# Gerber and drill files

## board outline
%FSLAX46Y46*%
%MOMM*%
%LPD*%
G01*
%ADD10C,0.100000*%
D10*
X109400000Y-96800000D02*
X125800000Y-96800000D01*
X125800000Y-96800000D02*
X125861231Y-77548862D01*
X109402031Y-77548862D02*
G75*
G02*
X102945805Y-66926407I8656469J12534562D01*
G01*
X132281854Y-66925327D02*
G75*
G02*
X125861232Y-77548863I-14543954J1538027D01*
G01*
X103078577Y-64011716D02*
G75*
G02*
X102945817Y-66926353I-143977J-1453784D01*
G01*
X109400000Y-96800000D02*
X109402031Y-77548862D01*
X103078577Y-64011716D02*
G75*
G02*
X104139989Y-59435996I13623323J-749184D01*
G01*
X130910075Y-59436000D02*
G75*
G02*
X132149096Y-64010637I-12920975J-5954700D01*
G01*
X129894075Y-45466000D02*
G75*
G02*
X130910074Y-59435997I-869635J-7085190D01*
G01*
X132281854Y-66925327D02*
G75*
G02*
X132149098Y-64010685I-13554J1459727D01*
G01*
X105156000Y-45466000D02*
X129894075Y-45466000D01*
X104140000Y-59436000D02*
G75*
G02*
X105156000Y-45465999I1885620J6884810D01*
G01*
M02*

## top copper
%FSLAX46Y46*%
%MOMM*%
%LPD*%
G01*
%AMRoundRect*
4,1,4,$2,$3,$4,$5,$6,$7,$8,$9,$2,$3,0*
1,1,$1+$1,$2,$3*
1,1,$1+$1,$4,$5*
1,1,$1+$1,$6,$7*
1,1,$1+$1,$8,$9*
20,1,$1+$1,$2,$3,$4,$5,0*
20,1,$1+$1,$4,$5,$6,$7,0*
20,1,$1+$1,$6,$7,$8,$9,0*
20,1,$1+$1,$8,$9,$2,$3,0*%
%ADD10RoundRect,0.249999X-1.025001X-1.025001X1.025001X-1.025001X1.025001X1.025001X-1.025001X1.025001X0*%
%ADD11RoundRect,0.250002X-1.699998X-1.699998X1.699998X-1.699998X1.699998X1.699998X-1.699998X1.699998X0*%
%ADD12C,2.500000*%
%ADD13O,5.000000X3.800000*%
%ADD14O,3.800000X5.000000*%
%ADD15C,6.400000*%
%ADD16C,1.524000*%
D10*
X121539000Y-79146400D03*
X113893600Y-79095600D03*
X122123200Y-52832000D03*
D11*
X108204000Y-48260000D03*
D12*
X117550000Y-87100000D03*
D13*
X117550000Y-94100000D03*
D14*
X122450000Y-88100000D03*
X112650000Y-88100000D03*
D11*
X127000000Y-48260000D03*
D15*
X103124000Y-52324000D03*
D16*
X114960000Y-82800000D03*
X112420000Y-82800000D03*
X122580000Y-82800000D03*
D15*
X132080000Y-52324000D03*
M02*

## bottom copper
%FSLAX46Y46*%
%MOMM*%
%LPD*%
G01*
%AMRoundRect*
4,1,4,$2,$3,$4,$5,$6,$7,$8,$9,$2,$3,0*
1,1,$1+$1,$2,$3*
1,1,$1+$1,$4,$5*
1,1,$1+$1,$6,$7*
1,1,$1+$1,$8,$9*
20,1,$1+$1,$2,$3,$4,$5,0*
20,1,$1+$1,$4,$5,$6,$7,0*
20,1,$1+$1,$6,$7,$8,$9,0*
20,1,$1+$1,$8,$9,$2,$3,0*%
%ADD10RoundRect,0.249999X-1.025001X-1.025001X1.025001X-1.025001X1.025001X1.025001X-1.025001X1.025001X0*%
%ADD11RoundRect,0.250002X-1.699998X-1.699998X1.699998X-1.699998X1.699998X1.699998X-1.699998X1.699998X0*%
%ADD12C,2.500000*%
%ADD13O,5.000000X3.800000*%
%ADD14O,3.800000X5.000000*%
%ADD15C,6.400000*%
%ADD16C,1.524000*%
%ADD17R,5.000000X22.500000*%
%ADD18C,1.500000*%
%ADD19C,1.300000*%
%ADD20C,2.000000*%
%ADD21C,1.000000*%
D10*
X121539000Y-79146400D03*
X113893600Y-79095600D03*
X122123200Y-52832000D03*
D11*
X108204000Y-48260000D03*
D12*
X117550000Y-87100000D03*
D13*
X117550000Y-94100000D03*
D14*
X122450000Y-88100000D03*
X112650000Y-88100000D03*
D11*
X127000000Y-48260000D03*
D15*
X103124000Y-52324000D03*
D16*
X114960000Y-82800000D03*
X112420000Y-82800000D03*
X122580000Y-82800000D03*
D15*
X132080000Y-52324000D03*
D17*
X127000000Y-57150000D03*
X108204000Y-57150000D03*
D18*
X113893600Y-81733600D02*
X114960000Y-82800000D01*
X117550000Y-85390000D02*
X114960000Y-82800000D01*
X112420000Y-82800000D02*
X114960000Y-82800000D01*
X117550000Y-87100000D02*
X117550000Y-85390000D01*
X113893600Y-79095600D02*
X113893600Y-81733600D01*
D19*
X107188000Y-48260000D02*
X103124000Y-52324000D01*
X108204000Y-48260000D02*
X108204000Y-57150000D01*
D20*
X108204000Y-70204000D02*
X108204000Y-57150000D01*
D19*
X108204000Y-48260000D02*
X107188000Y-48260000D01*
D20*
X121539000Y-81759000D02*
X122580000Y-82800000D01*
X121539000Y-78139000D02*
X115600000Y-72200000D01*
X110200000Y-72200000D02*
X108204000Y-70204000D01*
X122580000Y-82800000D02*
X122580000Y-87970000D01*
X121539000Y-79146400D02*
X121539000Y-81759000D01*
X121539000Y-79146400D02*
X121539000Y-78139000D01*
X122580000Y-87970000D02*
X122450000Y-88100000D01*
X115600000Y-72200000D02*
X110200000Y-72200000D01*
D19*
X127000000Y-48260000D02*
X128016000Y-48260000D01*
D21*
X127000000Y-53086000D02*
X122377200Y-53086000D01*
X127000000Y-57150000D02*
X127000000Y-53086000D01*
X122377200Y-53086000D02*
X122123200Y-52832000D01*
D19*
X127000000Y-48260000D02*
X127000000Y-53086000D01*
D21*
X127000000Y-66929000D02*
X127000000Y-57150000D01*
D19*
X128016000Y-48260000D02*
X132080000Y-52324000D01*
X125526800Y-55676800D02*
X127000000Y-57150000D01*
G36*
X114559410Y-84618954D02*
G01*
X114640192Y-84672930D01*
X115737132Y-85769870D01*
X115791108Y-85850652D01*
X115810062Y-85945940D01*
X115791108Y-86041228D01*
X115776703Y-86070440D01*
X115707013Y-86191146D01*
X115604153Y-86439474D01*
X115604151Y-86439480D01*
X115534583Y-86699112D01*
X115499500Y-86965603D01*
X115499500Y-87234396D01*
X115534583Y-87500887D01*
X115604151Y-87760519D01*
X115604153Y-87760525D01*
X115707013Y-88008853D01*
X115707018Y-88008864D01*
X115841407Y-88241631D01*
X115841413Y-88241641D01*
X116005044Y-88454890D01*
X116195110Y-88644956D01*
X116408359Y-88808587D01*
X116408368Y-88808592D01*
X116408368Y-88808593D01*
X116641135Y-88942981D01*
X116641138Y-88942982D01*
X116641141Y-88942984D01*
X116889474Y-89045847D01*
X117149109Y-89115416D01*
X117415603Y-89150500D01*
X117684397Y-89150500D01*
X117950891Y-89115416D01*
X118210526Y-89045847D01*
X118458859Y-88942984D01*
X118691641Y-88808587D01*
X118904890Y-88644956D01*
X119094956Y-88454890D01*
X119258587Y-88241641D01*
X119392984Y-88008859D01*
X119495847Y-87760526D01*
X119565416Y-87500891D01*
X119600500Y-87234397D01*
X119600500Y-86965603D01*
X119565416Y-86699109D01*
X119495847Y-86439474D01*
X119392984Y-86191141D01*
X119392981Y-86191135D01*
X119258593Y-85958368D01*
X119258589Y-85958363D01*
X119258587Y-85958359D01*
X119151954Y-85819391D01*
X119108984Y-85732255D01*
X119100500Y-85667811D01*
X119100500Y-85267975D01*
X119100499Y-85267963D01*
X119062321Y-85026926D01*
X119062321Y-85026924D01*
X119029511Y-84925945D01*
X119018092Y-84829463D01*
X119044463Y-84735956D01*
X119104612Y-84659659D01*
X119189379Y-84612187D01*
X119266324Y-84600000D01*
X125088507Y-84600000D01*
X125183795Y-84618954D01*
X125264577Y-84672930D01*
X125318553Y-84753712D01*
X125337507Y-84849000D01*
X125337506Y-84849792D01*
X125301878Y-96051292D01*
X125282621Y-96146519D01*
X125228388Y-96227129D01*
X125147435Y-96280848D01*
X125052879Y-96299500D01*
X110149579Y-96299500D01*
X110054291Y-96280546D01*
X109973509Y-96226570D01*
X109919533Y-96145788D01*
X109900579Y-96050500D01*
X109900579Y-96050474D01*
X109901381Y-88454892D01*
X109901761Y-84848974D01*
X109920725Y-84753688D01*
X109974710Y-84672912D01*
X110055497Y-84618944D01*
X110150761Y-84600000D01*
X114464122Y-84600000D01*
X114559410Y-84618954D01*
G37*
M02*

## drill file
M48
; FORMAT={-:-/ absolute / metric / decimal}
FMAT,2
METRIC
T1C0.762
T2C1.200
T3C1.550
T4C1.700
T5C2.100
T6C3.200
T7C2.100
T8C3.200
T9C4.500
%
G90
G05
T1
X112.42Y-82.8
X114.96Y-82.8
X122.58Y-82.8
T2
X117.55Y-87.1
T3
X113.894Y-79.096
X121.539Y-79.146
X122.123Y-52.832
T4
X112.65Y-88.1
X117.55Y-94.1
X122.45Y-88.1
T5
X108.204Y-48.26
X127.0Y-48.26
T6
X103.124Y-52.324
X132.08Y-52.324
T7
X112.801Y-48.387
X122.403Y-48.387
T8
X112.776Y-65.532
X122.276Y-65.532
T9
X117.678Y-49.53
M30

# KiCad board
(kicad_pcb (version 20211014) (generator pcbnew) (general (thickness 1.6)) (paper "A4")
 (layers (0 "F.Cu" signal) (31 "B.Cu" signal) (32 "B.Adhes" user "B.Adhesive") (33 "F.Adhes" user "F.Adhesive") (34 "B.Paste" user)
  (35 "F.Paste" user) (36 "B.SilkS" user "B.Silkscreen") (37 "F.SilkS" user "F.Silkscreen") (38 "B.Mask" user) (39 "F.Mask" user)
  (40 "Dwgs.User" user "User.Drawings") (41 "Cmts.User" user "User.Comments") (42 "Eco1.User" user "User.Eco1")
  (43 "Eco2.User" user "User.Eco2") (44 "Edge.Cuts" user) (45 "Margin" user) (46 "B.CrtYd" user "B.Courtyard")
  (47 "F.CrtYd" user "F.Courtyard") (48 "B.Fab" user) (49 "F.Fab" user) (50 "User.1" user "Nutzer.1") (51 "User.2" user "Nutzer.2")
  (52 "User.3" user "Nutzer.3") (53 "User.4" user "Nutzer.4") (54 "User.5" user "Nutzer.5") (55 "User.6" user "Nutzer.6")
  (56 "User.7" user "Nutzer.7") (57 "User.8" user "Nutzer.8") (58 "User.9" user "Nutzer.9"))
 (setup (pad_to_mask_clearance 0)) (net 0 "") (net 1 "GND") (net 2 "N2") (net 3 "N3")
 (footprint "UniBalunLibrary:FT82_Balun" (layer "F.Cu") (at 117.602 65.532)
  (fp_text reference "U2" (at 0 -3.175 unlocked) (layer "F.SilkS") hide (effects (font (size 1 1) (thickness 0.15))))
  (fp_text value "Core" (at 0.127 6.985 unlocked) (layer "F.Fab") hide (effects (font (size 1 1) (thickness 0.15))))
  (pad "" np_thru_hole circle (at -4.826 0) (size 3.2 3.2) (drill 3.2) (layers *.Cu *.Mask))
  (pad "" np_thru_hole circle (at 4.6736 0) (size 3.2 3.2) (drill 3.2) (layers *.Cu *.Mask))
  (pad "1" thru_hole roundrect (at 3.937 13.6144) (size 2.55 2.55) (drill 1.55) (layers *.Cu *.Mask) (roundrect_rratio 0.098039)
   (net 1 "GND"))
  (pad "2" thru_hole roundrect (at -3.7084 13.5636) (size 2.55 2.55) (drill 1.55) (layers *.Cu *.Mask) (roundrect_rratio 0.098039)
   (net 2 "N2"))
  (pad "3" thru_hole roundrect (at 4.5212 -12.7) (size 2.55 2.55) (drill 1.55) (layers *.Cu *.Mask) (roundrect_rratio 0.098039) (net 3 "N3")))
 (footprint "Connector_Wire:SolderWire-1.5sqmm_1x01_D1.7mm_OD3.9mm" (layer "F.Cu") (at 108.204 48.26)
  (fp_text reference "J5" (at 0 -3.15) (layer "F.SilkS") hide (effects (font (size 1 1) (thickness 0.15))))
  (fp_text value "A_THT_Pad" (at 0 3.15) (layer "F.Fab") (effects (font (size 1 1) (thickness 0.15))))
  (pad "1" thru_hole roundrect (at 0 0) (size 3.9 3.9) (drill 2.1) (layers *.Cu *.Mask) (roundrect_rratio 0.064103) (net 1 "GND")))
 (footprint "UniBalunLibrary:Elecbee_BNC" (layer "F.Cu") (at 112.65 88.1)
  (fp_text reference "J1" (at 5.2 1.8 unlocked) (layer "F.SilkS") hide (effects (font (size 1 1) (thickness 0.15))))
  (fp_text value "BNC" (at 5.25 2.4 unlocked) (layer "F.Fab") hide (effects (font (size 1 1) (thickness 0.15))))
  (pad "1" thru_hole circle (at 4.9 -1) (size 2.5 2.5) (drill 1.2) (layers *.Cu *.Mask) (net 2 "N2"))
  (pad "2" thru_hole oval (at 4.9 6 90) (size 3.8 5) (drill 1.7) (layers *.Cu *.Mask) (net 1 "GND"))
  (pad "2" thru_hole oval (at 9.8 0) (size 3.8 5) (drill 1.7) (layers *.Cu *.Mask) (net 1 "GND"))
  (pad "2" thru_hole oval (at 0 0) (size 3.8 5) (drill 1.7) (layers *.Cu *.Mask) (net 1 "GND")))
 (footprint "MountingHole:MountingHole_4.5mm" (layer "F.Cu") (at 117.6782 49.53)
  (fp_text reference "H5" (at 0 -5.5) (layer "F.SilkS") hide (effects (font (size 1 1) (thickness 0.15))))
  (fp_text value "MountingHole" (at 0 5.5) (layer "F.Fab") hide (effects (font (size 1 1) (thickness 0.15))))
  (pad "" np_thru_hole circle (at 0 0) (size 4.5 4.5) (drill 4.5) (layers *.Cu *.Mask)))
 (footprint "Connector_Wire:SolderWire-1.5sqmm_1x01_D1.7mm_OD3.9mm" (layer "F.Cu") (at 127 48.26)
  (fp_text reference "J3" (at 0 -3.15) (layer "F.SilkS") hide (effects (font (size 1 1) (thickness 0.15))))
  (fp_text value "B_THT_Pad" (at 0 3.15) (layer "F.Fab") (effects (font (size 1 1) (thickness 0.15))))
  (pad "1" thru_hole roundrect (at 0 0) (size 3.9 3.9) (drill 2.1) (layers *.Cu *.Mask) (roundrect_rratio 0.064103) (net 3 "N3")))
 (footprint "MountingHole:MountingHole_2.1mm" (layer "F.Cu") (at 112.8014 48.387)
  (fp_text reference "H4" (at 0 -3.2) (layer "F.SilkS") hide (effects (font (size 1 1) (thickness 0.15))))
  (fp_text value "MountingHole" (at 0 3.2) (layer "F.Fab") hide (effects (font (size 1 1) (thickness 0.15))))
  (pad "" np_thru_hole circle (at 0 0) (size 2.1 2.1) (drill 2.1) (layers *.Cu *.Mask)))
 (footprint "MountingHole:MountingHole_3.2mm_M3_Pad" (layer "F.Cu") (at 103.124 52.324)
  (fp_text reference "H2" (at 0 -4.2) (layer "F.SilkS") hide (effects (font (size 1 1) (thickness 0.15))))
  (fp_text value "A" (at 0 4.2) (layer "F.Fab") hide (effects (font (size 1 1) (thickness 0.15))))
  (pad "1" thru_hole circle (at 0 0) (size 6.4 6.4) (drill 3.2) (layers *.Cu *.Mask) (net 1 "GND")))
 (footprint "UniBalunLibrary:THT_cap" (layer "F.Cu") (at 117.5 82.8)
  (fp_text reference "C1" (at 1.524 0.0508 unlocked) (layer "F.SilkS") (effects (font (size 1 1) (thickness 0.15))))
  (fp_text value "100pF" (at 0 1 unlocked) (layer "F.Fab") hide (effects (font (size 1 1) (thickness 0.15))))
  (pad "1" thru_hole circle (at -2.54 0) (size 1.524 1.524) (drill 0.762) (layers *.Cu *.Mask) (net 2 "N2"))
  (pad "1" thru_hole circle (at -5.08 0) (size 1.524 1.524) (drill 0.762) (layers *.Cu *.Mask) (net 2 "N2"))
  (pad "2" thru_hole circle (at 5.08 0) (size 1.524 1.524) (drill 0.762) (layers *.Cu *.Mask) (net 1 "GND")))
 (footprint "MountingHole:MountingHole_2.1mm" (layer "F.Cu") (at 122.4026 48.387)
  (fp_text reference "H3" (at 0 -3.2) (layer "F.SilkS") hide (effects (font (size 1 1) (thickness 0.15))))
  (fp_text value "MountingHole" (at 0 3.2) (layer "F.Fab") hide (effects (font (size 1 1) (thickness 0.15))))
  (pad "" np_thru_hole circle (at 0 0) (size 2.1 2.1) (drill 2.1) (layers *.Cu *.Mask)))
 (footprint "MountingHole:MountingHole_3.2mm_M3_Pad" (layer "F.Cu") (at 132.08 52.324)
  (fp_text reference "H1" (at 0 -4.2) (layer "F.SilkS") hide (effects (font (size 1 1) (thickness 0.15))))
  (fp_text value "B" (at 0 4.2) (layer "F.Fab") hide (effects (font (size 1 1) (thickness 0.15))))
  (pad "1" thru_hole circle (at 0 0) (size 6.4 6.4) (drill 3.2) (layers *.Cu *.Mask) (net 3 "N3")))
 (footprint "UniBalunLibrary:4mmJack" (layer "B.Cu") (at 127.254 56.896 90)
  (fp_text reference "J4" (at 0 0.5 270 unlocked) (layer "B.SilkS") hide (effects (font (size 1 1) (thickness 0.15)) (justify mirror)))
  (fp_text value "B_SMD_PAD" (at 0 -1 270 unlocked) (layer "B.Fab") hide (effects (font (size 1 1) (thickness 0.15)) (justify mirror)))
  (pad "1" smd rect (at -0.254 -0.254 90) (size 22.5 5) (layers "B.Cu" "B.Mask") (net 3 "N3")))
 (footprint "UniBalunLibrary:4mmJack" (layer "B.Cu") (at 108.458 56.896 90)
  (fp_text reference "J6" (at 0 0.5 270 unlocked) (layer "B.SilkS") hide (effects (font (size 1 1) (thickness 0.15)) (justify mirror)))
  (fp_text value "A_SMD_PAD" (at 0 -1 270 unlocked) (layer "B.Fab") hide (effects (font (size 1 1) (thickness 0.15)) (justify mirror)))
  (pad "1" smd rect (at -0.254 -0.254 90) (size 22.5 5) (layers "B.Cu" "B.Mask") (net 1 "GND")))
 (gr_line (start 109.4 96.8) (end 125.8 96.8) (layer "Edge.Cuts") (width 0.1))
 (gr_line (start 125.8 96.8) (end 125.861231 77.548862) (layer "Edge.Cuts") (width 0.1))
 (gr_arc (start 109.402031 77.548862) (mid 105.04112 72.92614) (end 102.945817 66.926406) (layer "Edge.Cuts") (width 0.1))
 (gr_arc (start 132.281854 66.925327) (mid 130.254542 72.952072) (end 125.861231 77.548862) (layer "Edge.Cuts") (width 0.1))
 (gr_arc (start 103.078577 64.011716) (mid 104.394 65.532) (end 102.945817 66.926406) (layer "Edge.Cuts") (width 0.1))
 (gr_line (start 109.4 96.8) (end 109.402031 77.548862) (layer "Edge.Cuts") (width 0.1))
 (gr_arc (start 103.078577 64.011716) (mid 103.410896 61.677837) (end 104.14 59.436) (layer "Edge.Cuts") (width 0.1))
 (gr_arc (start 130.910075 59.436) (mid 131.721418 61.671361) (end 132.149094 64.010637) (layer "Edge.Cuts") (width 0.1))
 (gr_arc (start 129.894075 45.466) (mid 136.144 52.033405) (end 130.910075 59.436) (layer "Edge.Cuts") (width 0.1))
 (gr_arc (start 132.281854 66.925327) (mid 130.81 65.532) (end 132.149094 64.010637) (layer "Edge.Cuts") (width 0.1))
 (gr_line (start 105.156 45.466) (end 129.894075 45.466) (layer "Edge.Cuts") (width 0.1))
 (gr_arc (start 104.14 59.436) (mid 98.906069 52.033405) (end 105.156 45.466) (layer "Edge.Cuts") (width 0.1))
 (segment (start 113.8936 81.7336) (end 114.96 82.8) (width 1.5) (layer "B.Cu") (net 2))
 (segment (start 117.55 85.39) (end 114.96 82.8) (width 1.5) (layer "B.Cu") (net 2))
 (segment (start 112.42 82.8) (end 114.96 82.8) (width 1.5) (layer "B.Cu") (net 2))
 (segment (start 117.55 87.1) (end 117.55 85.39) (width 1.5) (layer "B.Cu") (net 2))
 (segment (start 113.8936 79.0956) (end 113.8936 81.7336) (width 1.5) (layer "B.Cu") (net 2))
 (segment (start 107.188 48.26) (end 103.124 52.324) (width 1.3) (layer "B.Cu") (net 1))
 (segment (start 108.204 48.26) (end 108.204 57.15) (width 1.3) (layer "B.Cu") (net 1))
 (segment (start 108.204 70.204) (end 108.204 57.15) (width 2) (layer "B.Cu") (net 1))
 (segment (start 108.204 48.26) (end 107.188 48.26) (width 1.3) (layer "B.Cu") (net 1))
 (segment (start 121.539 81.759) (end 122.58 82.8) (width 2) (layer "B.Cu") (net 1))
 (segment (start 121.539 78.139) (end 115.6 72.2) (width 2) (layer "B.Cu") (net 1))
 (segment (start 110.2 72.2) (end 108.204 70.204) (width 2) (layer "B.Cu") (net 1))
 (segment (start 122.58 82.8) (end 122.58 87.97) (width 2) (layer "B.Cu") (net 1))
 (segment (start 121.539 79.1464) (end 121.539 81.759) (width 2) (layer "B.Cu") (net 1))
 (segment (start 121.539 79.1464) (end 121.539 78.139) (width 2) (layer "B.Cu") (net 1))
 (segment (start 122.58 87.97) (end 122.45 88.1) (width 2) (layer "B.Cu") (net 1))
 (segment (start 115.6 72.2) (end 110.2 72.2) (width 2) (layer "B.Cu") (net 1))
 (segment (start 127 48.26) (end 128.016 48.26) (width 1.3) (layer "B.Cu") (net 3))
 (segment (start 127 53.086) (end 122.3772 53.086) (width 1) (layer "B.Cu") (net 3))
 (segment (start 127 57.15) (end 127 53.086) (width 1) (layer "B.Cu") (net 3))
 (segment (start 122.3772 53.086) (end 122.1232 52.832) (width 1) (layer "B.Cu") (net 3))
 (segment (start 127 48.26) (end 127 53.086) (width 1.3) (layer "B.Cu") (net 3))
 (segment (start 127 66.929) (end 127 57.15) (width 1) (layer "B.Cu") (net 3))
 (segment (start 128.016 48.26) (end 132.08 52.324) (width 1.3) (layer "B.Cu") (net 3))
 (segment (start 125.5268 55.6768) (end 127 57.15) (width 1.3) (layer "B.Cu") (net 3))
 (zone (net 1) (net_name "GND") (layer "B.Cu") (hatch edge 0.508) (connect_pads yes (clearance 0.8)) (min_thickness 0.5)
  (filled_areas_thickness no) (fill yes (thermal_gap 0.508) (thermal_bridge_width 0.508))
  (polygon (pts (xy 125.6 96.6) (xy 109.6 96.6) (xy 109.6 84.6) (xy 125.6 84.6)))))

